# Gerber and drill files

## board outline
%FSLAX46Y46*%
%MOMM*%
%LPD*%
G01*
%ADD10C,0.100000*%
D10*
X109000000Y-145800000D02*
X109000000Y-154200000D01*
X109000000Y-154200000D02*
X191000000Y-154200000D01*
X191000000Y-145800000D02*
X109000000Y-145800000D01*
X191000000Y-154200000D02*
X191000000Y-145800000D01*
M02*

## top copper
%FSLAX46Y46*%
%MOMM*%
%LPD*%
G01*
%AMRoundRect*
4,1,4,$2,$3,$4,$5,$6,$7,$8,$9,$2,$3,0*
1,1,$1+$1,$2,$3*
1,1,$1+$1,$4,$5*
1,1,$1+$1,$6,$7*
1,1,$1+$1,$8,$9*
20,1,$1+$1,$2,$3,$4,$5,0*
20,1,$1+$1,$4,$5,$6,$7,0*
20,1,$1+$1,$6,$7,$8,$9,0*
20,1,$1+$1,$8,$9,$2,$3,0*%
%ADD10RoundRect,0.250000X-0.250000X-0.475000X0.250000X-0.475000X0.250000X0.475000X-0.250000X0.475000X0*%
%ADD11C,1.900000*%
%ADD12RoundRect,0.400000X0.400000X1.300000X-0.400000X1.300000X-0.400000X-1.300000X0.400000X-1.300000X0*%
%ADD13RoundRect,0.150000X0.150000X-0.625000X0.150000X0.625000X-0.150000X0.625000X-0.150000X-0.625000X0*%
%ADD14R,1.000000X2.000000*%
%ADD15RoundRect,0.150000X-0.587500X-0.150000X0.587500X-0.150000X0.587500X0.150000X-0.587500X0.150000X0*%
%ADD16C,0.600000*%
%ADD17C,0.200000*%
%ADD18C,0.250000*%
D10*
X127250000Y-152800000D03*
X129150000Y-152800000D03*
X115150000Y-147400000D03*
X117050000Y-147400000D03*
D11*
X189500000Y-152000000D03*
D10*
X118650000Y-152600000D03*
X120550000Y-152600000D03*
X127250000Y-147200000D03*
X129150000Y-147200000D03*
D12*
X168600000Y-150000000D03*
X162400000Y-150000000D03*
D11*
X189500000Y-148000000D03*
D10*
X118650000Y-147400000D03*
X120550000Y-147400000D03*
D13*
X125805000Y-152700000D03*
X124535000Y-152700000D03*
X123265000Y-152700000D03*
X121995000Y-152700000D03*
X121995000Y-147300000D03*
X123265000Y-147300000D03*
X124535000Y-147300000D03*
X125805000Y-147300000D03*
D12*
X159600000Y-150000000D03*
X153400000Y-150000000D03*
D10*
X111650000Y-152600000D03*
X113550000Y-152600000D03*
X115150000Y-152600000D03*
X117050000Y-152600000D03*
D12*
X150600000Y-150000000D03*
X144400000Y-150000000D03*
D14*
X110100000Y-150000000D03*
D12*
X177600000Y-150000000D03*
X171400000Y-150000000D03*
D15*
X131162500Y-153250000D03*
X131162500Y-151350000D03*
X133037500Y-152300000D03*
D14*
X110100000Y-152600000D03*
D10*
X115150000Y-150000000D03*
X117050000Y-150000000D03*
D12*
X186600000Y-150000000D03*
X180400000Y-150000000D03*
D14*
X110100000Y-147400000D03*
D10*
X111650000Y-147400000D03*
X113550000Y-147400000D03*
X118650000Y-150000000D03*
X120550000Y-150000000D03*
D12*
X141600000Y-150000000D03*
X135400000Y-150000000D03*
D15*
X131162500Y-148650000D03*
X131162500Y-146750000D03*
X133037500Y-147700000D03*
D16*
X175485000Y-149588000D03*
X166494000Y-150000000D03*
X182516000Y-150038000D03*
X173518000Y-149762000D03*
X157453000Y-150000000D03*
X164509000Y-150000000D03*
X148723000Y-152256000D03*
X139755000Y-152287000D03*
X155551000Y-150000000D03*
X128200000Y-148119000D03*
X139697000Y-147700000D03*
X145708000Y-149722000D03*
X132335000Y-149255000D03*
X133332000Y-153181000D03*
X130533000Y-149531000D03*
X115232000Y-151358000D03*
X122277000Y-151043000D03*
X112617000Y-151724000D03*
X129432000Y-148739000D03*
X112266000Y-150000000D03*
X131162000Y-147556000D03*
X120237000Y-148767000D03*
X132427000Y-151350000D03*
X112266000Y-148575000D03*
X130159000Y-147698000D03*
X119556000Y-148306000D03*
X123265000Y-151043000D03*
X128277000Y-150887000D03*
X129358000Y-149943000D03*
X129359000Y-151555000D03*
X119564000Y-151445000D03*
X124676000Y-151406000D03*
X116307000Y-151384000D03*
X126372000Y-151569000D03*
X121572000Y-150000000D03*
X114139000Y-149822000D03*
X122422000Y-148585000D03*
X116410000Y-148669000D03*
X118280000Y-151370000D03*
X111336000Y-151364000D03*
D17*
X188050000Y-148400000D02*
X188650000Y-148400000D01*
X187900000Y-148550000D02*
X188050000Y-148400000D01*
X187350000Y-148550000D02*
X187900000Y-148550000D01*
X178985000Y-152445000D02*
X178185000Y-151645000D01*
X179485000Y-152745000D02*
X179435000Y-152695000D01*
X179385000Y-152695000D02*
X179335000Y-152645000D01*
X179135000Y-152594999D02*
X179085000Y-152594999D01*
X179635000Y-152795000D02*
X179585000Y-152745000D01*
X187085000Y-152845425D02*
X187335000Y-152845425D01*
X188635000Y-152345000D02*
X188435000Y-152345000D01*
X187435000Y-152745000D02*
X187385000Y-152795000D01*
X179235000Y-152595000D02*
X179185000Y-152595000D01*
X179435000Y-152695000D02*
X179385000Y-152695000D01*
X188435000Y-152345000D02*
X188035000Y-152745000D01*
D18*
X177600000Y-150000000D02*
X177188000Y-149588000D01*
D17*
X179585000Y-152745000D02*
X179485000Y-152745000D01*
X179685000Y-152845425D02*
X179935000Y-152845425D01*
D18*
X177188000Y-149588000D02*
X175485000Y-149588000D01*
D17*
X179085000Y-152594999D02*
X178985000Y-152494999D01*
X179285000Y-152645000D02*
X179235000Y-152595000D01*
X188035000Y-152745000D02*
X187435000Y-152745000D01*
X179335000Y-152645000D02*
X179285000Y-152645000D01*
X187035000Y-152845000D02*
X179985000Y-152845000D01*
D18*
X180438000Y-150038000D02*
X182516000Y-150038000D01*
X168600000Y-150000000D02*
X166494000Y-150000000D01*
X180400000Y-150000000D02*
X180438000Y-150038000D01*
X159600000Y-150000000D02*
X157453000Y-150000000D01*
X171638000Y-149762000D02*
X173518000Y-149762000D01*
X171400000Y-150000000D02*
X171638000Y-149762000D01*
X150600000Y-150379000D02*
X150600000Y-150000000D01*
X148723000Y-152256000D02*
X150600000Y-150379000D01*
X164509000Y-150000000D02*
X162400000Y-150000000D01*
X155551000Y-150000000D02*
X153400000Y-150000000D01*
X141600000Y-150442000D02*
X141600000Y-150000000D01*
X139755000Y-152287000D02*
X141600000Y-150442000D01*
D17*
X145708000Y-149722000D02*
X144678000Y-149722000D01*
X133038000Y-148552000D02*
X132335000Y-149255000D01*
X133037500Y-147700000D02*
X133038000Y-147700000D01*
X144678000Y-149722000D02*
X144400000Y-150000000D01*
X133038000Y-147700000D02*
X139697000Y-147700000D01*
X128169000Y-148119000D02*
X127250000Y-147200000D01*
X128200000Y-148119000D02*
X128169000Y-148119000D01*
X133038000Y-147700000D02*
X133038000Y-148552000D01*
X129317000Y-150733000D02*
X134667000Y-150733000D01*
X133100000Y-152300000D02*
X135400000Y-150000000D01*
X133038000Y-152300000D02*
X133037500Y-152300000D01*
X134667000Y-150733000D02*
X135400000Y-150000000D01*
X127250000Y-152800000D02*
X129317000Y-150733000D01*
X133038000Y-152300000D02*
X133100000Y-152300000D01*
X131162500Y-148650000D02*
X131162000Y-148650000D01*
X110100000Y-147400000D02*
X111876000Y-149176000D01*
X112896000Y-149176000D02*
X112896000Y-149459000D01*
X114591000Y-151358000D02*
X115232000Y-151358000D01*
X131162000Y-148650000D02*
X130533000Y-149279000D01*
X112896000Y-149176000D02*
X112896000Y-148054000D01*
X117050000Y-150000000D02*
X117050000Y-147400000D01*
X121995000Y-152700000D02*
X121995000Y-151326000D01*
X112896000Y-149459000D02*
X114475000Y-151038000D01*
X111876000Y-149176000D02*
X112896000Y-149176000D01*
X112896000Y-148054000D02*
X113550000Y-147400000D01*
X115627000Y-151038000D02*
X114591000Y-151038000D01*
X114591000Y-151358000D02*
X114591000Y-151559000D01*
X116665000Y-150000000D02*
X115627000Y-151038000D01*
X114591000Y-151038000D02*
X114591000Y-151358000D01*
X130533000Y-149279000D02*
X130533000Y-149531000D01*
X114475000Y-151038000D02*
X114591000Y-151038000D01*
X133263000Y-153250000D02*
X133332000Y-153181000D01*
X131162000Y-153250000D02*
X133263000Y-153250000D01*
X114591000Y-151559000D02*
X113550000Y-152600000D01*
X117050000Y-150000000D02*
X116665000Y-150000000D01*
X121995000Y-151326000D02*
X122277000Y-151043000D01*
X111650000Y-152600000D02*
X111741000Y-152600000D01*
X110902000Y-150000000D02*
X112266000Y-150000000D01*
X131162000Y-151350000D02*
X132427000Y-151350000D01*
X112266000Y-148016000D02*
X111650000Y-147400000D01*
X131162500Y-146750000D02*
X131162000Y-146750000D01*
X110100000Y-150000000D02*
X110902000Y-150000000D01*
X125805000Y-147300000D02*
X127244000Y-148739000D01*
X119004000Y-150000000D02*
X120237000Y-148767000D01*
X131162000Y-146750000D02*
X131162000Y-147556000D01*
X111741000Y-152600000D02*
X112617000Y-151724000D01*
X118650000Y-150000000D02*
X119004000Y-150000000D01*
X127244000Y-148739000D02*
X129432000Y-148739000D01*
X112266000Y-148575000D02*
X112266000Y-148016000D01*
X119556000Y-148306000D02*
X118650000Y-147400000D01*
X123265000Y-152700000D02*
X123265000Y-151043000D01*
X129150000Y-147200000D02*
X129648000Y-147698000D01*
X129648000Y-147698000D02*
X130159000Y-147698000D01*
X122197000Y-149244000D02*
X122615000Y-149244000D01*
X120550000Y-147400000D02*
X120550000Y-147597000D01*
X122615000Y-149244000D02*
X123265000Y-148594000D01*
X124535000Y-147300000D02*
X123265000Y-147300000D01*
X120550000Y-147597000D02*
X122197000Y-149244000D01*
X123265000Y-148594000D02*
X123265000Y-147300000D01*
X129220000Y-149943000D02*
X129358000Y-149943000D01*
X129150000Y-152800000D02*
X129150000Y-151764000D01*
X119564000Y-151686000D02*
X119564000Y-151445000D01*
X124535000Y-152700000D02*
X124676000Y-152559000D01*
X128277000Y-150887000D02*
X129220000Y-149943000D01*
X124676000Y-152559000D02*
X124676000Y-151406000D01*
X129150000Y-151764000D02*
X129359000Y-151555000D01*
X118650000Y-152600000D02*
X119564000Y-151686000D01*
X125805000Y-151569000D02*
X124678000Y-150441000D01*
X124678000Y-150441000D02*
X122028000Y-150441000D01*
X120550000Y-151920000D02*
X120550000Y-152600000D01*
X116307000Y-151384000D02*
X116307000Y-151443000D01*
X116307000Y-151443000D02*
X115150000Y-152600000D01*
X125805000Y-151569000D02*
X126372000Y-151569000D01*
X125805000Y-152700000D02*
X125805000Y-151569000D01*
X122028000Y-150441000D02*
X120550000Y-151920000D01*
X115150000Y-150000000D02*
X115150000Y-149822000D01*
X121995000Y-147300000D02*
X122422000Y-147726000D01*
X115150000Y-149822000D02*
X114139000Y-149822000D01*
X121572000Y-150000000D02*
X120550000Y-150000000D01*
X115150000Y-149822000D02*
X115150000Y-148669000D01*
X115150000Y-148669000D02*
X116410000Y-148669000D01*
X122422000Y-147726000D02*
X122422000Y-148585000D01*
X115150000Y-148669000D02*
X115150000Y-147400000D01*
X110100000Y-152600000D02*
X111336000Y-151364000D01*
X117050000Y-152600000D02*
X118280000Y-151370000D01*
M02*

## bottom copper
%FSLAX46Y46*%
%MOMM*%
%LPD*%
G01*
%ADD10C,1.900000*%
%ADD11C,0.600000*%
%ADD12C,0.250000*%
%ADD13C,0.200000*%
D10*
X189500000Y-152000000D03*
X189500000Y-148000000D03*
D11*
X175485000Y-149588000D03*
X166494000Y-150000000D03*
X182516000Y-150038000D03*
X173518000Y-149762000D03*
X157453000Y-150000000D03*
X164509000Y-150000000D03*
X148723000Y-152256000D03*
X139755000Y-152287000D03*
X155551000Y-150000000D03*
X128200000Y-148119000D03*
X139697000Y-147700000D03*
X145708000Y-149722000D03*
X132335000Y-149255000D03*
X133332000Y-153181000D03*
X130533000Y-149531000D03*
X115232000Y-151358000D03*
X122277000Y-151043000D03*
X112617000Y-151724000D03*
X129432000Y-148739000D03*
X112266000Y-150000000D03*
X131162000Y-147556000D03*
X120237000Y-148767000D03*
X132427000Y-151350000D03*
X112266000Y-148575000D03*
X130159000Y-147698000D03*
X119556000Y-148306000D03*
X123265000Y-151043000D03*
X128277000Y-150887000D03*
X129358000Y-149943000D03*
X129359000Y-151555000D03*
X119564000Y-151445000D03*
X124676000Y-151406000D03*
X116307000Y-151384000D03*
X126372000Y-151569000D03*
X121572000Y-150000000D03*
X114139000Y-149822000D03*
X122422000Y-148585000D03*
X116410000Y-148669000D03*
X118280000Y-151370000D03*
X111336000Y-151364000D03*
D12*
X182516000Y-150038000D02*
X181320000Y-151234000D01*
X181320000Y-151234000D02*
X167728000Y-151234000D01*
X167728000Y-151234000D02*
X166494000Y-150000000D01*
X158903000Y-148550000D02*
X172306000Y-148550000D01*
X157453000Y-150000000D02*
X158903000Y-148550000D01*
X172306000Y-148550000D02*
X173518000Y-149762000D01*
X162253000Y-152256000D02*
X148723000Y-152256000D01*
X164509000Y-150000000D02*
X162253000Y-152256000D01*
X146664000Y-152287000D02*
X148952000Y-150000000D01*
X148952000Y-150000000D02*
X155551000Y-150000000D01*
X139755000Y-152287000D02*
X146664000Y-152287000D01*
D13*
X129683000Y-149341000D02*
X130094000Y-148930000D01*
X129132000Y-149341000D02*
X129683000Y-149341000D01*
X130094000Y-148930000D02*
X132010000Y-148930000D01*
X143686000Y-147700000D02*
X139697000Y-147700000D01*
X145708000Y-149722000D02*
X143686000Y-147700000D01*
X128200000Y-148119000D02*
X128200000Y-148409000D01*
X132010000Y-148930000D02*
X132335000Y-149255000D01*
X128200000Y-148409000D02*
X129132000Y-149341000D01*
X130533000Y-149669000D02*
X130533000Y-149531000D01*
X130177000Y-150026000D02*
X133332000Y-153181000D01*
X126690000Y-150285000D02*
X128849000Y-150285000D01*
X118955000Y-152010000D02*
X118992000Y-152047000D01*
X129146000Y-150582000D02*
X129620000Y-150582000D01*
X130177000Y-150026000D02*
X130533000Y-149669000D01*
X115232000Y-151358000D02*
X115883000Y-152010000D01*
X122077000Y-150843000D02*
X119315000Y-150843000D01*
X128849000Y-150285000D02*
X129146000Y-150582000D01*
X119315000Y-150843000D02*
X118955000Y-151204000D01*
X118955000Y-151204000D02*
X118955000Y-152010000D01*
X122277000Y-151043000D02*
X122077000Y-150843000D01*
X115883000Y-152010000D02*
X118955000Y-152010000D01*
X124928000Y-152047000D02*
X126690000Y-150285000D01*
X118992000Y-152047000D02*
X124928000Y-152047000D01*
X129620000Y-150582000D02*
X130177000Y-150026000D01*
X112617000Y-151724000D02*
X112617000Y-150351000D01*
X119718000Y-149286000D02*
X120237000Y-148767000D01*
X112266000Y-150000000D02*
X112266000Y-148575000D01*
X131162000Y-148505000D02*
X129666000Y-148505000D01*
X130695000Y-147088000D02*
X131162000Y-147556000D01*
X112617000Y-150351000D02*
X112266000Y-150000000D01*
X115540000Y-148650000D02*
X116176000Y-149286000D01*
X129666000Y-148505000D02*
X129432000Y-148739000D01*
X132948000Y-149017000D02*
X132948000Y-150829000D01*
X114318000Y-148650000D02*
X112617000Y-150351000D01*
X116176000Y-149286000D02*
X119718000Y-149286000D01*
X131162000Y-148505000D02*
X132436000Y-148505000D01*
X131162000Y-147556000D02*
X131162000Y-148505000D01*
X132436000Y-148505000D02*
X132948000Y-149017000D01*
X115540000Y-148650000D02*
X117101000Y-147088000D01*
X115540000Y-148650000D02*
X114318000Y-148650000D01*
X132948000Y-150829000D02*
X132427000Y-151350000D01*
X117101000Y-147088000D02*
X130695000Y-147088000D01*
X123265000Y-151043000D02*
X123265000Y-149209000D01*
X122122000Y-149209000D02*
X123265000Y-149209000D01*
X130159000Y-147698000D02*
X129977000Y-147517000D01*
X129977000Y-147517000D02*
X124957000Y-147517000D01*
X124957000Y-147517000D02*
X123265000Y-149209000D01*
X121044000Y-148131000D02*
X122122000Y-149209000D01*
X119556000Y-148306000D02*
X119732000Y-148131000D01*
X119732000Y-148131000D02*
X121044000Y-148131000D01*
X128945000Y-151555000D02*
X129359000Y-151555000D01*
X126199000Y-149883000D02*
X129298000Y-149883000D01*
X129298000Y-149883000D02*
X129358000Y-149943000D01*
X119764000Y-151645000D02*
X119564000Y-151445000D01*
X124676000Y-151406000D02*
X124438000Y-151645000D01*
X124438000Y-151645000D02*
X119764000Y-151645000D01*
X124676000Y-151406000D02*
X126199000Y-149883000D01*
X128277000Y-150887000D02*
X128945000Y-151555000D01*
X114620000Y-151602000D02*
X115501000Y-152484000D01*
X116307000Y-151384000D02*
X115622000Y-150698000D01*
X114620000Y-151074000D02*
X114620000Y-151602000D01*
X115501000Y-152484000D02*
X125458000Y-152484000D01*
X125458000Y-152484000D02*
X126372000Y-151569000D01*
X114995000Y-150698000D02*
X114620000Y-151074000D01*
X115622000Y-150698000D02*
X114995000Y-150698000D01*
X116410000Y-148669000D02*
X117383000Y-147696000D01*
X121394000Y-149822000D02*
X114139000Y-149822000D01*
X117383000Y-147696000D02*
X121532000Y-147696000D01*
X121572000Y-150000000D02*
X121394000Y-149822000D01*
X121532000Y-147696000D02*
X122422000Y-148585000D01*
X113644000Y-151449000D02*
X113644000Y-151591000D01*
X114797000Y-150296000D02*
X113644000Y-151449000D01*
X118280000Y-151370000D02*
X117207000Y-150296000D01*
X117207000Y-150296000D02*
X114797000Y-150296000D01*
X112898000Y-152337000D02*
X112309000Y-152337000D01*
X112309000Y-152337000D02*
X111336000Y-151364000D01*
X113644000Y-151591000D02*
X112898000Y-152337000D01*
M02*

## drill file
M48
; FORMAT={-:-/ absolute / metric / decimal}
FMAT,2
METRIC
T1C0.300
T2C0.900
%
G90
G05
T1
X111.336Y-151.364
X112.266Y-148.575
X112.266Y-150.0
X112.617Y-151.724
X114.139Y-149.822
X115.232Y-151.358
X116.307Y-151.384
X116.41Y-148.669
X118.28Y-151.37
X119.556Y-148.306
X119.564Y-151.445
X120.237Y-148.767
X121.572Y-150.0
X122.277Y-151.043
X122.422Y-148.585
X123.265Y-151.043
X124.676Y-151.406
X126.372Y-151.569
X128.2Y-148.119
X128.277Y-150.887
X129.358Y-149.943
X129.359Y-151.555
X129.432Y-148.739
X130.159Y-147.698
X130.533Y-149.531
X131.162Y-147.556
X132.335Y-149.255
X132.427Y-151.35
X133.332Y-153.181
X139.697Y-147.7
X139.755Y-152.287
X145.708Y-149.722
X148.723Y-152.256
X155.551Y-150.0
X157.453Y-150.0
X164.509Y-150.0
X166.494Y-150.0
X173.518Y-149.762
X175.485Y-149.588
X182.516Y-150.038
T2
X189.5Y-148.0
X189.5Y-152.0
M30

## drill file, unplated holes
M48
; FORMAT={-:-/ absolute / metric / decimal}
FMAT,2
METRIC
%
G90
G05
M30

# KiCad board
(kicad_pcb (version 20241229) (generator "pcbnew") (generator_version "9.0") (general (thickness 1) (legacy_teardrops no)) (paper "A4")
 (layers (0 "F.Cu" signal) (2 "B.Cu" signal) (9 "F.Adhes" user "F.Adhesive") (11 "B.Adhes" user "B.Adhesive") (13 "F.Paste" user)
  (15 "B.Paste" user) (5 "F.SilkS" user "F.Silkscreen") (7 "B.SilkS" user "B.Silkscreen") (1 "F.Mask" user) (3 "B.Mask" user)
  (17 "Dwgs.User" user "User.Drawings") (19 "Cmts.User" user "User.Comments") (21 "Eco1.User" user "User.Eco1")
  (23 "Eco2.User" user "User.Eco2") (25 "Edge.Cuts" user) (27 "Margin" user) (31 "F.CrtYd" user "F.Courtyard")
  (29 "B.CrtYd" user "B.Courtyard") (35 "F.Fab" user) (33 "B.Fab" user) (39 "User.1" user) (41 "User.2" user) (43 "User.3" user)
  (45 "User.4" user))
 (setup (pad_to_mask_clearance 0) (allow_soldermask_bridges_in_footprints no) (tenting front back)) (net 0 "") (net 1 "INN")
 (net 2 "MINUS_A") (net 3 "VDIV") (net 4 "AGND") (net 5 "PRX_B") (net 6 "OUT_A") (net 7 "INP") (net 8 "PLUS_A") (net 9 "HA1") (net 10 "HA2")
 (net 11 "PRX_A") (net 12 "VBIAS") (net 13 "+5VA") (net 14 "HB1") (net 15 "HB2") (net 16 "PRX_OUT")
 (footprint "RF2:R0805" (layer "F.Cu") (at 128.199999 152.8)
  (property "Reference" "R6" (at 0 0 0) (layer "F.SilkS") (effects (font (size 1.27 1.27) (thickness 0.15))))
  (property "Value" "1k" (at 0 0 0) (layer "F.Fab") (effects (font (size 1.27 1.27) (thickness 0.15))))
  (pad "1" smd roundrect (at -0.949999 0) (size 1 1.45) (layers "F.Cu" "F.Mask" "F.Paste") (roundrect_rratio 0.25) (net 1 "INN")
   (thermal_bridge_angle 45))
  (pad "2" smd roundrect (at 0.950001 0) (size 1 1.45) (layers "F.Cu" "F.Mask" "F.Paste") (roundrect_rratio 0.25) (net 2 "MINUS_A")
   (thermal_bridge_angle 45)))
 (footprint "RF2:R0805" (layer "F.Cu") (at 116.1 147.4)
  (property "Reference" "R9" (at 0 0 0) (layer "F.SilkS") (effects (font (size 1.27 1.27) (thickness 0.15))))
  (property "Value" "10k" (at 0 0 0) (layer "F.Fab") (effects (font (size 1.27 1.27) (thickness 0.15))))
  (pad "1" smd roundrect (at -0.95 0) (size 1 1.45) (layers "F.Cu" "F.Mask" "F.Paste") (roundrect_rratio 0.25) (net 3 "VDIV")
   (thermal_bridge_angle 45))
  (pad "2" smd roundrect (at 0.95 0) (size 1 1.45) (layers "F.Cu" "F.Mask" "F.Paste") (roundrect_rratio 0.25) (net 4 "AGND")
   (thermal_bridge_angle 45)))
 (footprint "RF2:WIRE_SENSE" (layer "F.Cu") (at 189.5 152)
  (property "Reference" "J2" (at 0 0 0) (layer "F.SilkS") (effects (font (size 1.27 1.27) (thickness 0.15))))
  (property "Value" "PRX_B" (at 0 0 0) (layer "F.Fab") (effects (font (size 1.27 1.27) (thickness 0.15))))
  (pad "1" thru_hole circle (at 0 0) (size 1.9 1.9) (drill 0.9) (layers "*.Cu" "*.Mask") (remove_unused_layers no) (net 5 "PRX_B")))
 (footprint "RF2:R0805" (layer "F.Cu") (at 119.6 152.6)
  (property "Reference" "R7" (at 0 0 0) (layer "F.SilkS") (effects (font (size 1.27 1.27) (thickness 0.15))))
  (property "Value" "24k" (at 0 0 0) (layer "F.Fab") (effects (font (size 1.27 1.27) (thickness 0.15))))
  (pad "1" smd roundrect (at -0.95 0) (size 1 1.45) (layers "F.Cu" "F.Mask" "F.Paste") (roundrect_rratio 0.25) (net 2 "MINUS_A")
   (thermal_bridge_angle 45))
  (pad "2" smd roundrect (at 0.95 0) (size 1 1.45) (layers "F.Cu" "F.Mask" "F.Paste") (roundrect_rratio 0.25) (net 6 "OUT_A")
   (thermal_bridge_angle 45)))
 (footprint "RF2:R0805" (layer "F.Cu") (at 128.199999 147.2)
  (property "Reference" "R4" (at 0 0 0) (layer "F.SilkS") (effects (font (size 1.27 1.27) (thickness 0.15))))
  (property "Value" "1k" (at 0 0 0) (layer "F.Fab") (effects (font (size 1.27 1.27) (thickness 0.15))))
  (pad "1" smd roundrect (at -0.949999 0) (size 1 1.45) (layers "F.Cu" "F.Mask" "F.Paste") (roundrect_rratio 0.25) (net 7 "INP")
   (thermal_bridge_angle 45))
  (pad "2" smd roundrect (at 0.950001 0) (size 1 1.45) (layers "F.Cu" "F.Mask" "F.Paste") (roundrect_rratio 0.25) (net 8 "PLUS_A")
   (thermal_bridge_angle 45)))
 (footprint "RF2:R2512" (layer "F.Cu") (at 165.5 150 180)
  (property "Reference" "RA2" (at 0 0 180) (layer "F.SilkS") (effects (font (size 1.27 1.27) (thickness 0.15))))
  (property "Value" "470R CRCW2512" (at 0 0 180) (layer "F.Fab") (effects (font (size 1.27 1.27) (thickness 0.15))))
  (pad "1" smd roundrect (at -3.1 0 180) (size 1.6 3.4) (layers "F.Cu" "F.Mask" "F.Paste") (roundrect_rratio 0.25) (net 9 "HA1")
   (thermal_bridge_angle 45))
  (pad "2" smd roundrect (at 3.1 0 180) (size 1.6 3.4) (layers "F.Cu" "F.Mask" "F.Paste") (roundrect_rratio 0.25) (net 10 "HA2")
   (thermal_bridge_angle 45)))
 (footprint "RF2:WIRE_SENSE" (layer "F.Cu") (at 189.5 148)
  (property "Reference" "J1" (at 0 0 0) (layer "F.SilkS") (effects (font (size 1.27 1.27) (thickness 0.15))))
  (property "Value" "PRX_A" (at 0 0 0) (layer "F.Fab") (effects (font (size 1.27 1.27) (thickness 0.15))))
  (pad "1" thru_hole circle (at 0 0) (size 1.9 1.9) (drill 0.9) (layers "*.Cu" "*.Mask") (remove_unused_layers no) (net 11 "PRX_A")))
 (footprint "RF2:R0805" (layer "F.Cu") (at 119.6 147.4)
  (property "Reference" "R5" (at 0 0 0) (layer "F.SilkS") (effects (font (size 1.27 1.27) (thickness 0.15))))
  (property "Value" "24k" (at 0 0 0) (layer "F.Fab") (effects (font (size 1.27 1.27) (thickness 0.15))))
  (pad "1" smd roundrect (at -0.95 0) (size 1 1.45) (layers "F.Cu" "F.Mask" "F.Paste") (roundrect_rratio 0.25) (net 8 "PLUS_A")
   (thermal_bridge_angle 45))
  (pad "2" smd roundrect (at 0.95 0) (size 1 1.45) (layers "F.Cu" "F.Mask" "F.Paste") (roundrect_rratio 0.25) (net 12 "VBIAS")
   (thermal_bridge_angle 45)))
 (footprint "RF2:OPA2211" (layer "F.Cu") (at 123.9 150 90)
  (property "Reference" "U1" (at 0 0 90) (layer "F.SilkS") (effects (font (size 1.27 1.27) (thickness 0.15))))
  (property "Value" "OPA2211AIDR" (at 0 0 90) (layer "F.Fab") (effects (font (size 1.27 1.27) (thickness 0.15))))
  (pad "1" smd roundrect (at -2.7 1.905 90) (size 1.55 0.6) (layers "F.Cu" "F.Mask" "F.Paste") (roundrect_rratio 0.25) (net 6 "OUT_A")
   (thermal_bridge_angle 45))
  (pad "2" smd roundrect (at -2.7 0.635 90) (size 1.55 0.6) (layers "F.Cu" "F.Mask" "F.Paste") (roundrect_rratio 0.25) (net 2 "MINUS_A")
   (thermal_bridge_angle 45))
  (pad "3" smd roundrect (at -2.7 -0.635 90) (size 1.55 0.6) (layers "F.Cu" "F.Mask" "F.Paste") (roundrect_rratio 0.25) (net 8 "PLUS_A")
   (thermal_bridge_angle 45))
  (pad "4" smd roundrect (at -2.7 -1.905 90) (size 1.55 0.6) (layers "F.Cu" "F.Mask" "F.Paste") (roundrect_rratio 0.25) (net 4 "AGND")
   (thermal_bridge_angle 45))
  (pad "5" smd roundrect (at 2.7 -1.905 90) (size 1.55 0.6) (layers "F.Cu" "F.Mask" "F.Paste") (roundrect_rratio 0.25) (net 3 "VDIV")
   (thermal_bridge_angle 45))
  (pad "6" smd roundrect (at 2.7 -0.635 90) (size 1.55 0.6) (layers "F.Cu" "F.Mask" "F.Paste") (roundrect_rratio 0.25) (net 12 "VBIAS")
   (thermal_bridge_angle 45))
  (pad "7" smd roundrect (at 2.7 0.635 90) (size 1.55 0.6) (layers "F.Cu" "F.Mask" "F.Paste") (roundrect_rratio 0.25) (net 12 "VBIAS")
   (thermal_bridge_angle 45))
  (pad "8" smd roundrect (at 2.7 1.905 90) (size 1.55 0.6) (layers "F.Cu" "F.Mask" "F.Paste") (roundrect_rratio 0.25) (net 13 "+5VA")
   (thermal_bridge_angle 45)))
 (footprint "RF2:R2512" (layer "F.Cu") (at 156.5 150 180)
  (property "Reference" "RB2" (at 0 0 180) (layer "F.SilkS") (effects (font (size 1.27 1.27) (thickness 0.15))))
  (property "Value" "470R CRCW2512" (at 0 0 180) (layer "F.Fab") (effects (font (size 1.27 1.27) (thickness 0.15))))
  (pad "1" smd roundrect (at -3.1 0 180) (size 1.6 3.4) (layers "F.Cu" "F.Mask" "F.Paste") (roundrect_rratio 0.25) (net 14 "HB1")
   (thermal_bridge_angle 45))
  (pad "2" smd roundrect (at 3.1 0 180) (size 1.6 3.4) (layers "F.Cu" "F.Mask" "F.Paste") (roundrect_rratio 0.25) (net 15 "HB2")
   (thermal_bridge_angle 45)))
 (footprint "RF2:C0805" (layer "F.Cu") (at 112.6 152.6)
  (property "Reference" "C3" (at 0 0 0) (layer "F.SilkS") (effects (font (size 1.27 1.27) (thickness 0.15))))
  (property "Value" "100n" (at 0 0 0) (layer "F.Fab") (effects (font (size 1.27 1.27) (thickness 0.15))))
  (pad "1" smd roundrect (at -0.95 0) (size 1 1.45) (layers "F.Cu" "F.Mask" "F.Paste") (roundrect_rratio 0.25) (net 13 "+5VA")
   (thermal_bridge_angle 45))
  (pad "2" smd roundrect (at 0.95 0) (size 1 1.45) (layers "F.Cu" "F.Mask" "F.Paste") (roundrect_rratio 0.25) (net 4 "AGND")
   (thermal_bridge_angle 45)))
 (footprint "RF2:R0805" (layer "F.Cu") (at 116.1 152.6)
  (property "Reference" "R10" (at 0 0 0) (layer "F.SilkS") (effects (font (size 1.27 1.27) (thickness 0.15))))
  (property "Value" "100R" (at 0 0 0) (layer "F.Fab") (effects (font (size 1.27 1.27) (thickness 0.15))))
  (pad "1" smd roundrect (at -0.95 0) (size 1 1.45) (layers "F.Cu" "F.Mask" "F.Paste") (roundrect_rratio 0.25) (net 6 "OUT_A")
   (thermal_bridge_angle 45))
  (pad "2" smd roundrect (at 0.95 0) (size 1 1.45) (layers "F.Cu" "F.Mask" "F.Paste") (roundrect_rratio 0.25) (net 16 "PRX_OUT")
   (thermal_bridge_angle 45)))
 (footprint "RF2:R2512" (layer "F.Cu") (at 147.5 150 180)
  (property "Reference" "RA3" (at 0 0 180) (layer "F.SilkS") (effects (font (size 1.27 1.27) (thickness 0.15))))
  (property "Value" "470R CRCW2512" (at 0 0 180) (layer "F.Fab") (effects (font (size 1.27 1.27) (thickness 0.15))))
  (pad "1" smd roundrect (at -3.1 0 180) (size 1.6 3.4) (layers "F.Cu" "F.Mask" "F.Paste") (roundrect_rratio 0.25) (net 10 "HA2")
   (thermal_bridge_angle 45))
  (pad "2" smd roundrect (at 3.1 0 180) (size 1.6 3.4) (layers "F.Cu" "F.Mask" "F.Paste") (roundrect_rratio 0.25) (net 7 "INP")
   (thermal_bridge_angle 45)))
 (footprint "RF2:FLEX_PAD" (layer "F.Cu") (at 110.1 150)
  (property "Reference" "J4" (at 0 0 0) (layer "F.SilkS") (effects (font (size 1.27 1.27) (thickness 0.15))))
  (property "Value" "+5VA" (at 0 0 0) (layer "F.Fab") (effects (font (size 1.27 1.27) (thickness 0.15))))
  (pad "1" smd rect (at 0 0) (size 1 2) (layers "F.Cu" "F.Mask" "F.Paste") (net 13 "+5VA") (thermal_bridge_angle 45)))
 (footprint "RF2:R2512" (layer "F.Cu") (at 174.5 150 180)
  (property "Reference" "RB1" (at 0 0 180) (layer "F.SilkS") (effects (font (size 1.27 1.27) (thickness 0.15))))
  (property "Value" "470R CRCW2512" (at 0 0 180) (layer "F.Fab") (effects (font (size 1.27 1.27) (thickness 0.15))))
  (pad "1" smd roundrect (at -3.1 0 180) (size 1.6 3.4) (layers "F.Cu" "F.Mask" "F.Paste") (roundrect_rratio 0.25) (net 5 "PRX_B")
   (thermal_bridge_angle 45))
  (pad "2" smd roundrect (at 3.1 0 180) (size 1.6 3.4) (layers "F.Cu" "F.Mask" "F.Paste") (roundrect_rratio 0.25) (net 14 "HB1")
   (thermal_bridge_angle 45)))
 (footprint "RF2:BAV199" (layer "F.Cu") (at 132.1 152.3)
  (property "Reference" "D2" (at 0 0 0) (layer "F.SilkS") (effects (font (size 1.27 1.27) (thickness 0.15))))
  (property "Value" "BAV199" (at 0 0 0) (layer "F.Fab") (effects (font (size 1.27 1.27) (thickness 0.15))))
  (pad "1" smd roundrect (at -0.9375 0.95) (size 1.475 0.6) (layers "F.Cu" "F.Mask" "F.Paste") (roundrect_rratio 0.25) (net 4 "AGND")
   (thermal_bridge_angle 45))
  (pad "2" smd roundrect (at -0.9375 -0.95) (size 1.475 0.6) (layers "F.Cu" "F.Mask" "F.Paste") (roundrect_rratio 0.25) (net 13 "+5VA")
   (thermal_bridge_angle 45))
  (pad "3" smd roundrect (at 0.9375 0) (size 1.475 0.6) (layers "F.Cu" "F.Mask" "F.Paste") (roundrect_rratio 0.25) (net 1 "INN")
   (thermal_bridge_angle 45)))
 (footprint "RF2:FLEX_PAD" (layer "F.Cu") (at 110.1 152.6)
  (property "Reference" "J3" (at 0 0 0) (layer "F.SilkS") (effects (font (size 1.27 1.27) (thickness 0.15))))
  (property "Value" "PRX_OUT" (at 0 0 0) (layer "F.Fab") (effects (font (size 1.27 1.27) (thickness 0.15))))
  (pad "1" smd rect (at 0 0) (size 1 2) (layers "F.Cu" "F.Mask" "F.Paste") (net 16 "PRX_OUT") (thermal_bridge_angle 45)))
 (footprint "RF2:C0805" (layer "F.Cu") (at 116.1 150)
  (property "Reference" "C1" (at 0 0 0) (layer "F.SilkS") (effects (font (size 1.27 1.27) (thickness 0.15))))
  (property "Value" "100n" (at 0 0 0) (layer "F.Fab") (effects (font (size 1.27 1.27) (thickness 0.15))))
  (pad "1" smd roundrect (at -0.95 0) (size 1 1.45) (layers "F.Cu" "F.Mask" "F.Paste") (roundrect_rratio 0.25) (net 3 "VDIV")
   (thermal_bridge_angle 45))
  (pad "2" smd roundrect (at 0.95 0) (size 1 1.45) (layers "F.Cu" "F.Mask" "F.Paste") (roundrect_rratio 0.25) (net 4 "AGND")
   (thermal_bridge_angle 45)))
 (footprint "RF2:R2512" (layer "F.Cu") (at 183.5 150 180)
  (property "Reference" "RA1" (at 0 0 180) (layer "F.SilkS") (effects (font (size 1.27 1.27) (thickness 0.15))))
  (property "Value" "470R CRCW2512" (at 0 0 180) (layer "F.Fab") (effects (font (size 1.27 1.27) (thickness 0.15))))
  (pad "1" smd roundrect (at -3.1 0 180) (size 1.6 3.4) (layers "F.Cu" "F.Mask" "F.Paste") (roundrect_rratio 0.25) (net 11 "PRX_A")
   (thermal_bridge_angle 45))
  (pad "2" smd roundrect (at 3.1 0 180) (size 1.6 3.4) (layers "F.Cu" "F.Mask" "F.Paste") (roundrect_rratio 0.25) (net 9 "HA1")
   (thermal_bridge_angle 45)))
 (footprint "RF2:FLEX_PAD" (layer "F.Cu") (at 110.1 147.4)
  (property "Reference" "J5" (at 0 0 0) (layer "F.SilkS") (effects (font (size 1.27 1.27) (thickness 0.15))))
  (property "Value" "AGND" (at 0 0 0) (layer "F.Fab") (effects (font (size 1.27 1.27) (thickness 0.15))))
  (pad "1" smd rect (at 0 0) (size 1 2) (layers "F.Cu" "F.Mask" "F.Paste") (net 4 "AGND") (thermal_bridge_angle 45)))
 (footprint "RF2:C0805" (layer "F.Cu") (at 112.6 147.4)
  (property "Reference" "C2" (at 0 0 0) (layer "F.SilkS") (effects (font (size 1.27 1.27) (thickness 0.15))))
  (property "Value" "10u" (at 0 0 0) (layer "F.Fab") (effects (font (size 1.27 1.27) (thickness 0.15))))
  (pad "1" smd roundrect (at -0.95 0) (size 1 1.45) (layers "F.Cu" "F.Mask" "F.Paste") (roundrect_rratio 0.25) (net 13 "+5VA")
   (thermal_bridge_angle 45))
  (pad "2" smd roundrect (at 0.95 0) (size 1 1.45) (layers "F.Cu" "F.Mask" "F.Paste") (roundrect_rratio 0.25) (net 4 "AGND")
   (thermal_bridge_angle 45)))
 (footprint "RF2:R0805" (layer "F.Cu") (at 119.6 150)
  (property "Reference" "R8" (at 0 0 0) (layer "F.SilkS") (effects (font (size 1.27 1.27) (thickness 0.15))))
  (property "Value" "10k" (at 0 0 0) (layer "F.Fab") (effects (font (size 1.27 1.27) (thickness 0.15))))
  (pad "1" smd roundrect (at -0.95 0) (size 1 1.45) (layers "F.Cu" "F.Mask" "F.Paste") (roundrect_rratio 0.25) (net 13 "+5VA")
   (thermal_bridge_angle 45))
  (pad "2" smd roundrect (at 0.95 0) (size 1 1.45) (layers "F.Cu" "F.Mask" "F.Paste") (roundrect_rratio 0.25) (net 3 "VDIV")
   (thermal_bridge_angle 45)))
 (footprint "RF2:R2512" (layer "F.Cu") (at 138.5 150 180)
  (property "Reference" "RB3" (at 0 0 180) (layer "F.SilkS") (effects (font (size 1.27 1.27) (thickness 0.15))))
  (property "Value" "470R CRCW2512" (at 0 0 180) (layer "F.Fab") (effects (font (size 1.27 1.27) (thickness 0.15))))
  (pad "1" smd roundrect (at -3.1 0 180) (size 1.6 3.4) (layers "F.Cu" "F.Mask" "F.Paste") (roundrect_rratio 0.25) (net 15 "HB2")
   (thermal_bridge_angle 45))
  (pad "2" smd roundrect (at 3.1 0 180) (size 1.6 3.4) (layers "F.Cu" "F.Mask" "F.Paste") (roundrect_rratio 0.25) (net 1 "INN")
   (thermal_bridge_angle 45)))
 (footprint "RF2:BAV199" (layer "F.Cu") (at 132.1 147.7)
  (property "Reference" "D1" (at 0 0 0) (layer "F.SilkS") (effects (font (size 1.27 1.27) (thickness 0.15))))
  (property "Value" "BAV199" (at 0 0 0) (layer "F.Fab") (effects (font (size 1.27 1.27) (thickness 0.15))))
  (pad "1" smd roundrect (at -0.9375 0.95) (size 1.475 0.6) (layers "F.Cu" "F.Mask" "F.Paste") (roundrect_rratio 0.25) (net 4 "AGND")
   (thermal_bridge_angle 45))
  (pad "2" smd roundrect (at -0.9375 -0.95) (size 1.475 0.6) (layers "F.Cu" "F.Mask" "F.Paste") (roundrect_rratio 0.25) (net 13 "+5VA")
   (thermal_bridge_angle 45))
  (pad "3" smd roundrect (at 0.9375 0) (size 1.475 0.6) (layers "F.Cu" "F.Mask" "F.Paste") (roundrect_rratio 0.25) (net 7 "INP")
   (thermal_bridge_angle 45)))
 (gr_line (start 109 145.8) (end 109 154.2) (stroke (width 0.1) (type default)) (layer "Edge.Cuts"))
 (gr_line (start 109 154.2) (end 191 154.2) (stroke (width 0.1) (type default)) (layer "Edge.Cuts"))
 (gr_line (start 191 145.8) (end 109 145.8) (stroke (width 0.1) (type default)) (layer "Edge.Cuts"))
 (gr_line (start 191 154.2) (end 191 145.8) (stroke (width 0.1) (type default)) (layer "Edge.Cuts"))
 (segment (start 188.05 148.4) (end 188.65 148.4) (width 0.2) (layer "F.Cu") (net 11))
 (segment (start 187.9 148.55) (end 188.05 148.4) (width 0.2) (layer "F.Cu") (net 11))
 (segment (start 187.35 148.55) (end 187.9 148.55) (width 0.2) (layer "F.Cu") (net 11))
 (segment (start 178.985 152.445) (end 178.185 151.645) (width 0.2) (layer "F.Cu") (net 5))
 (segment (start 179.485 152.745) (end 179.435 152.695) (width 0.2) (layer "F.Cu") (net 5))
 (segment (start 179.385 152.695) (end 179.335 152.645) (width 0.2) (layer "F.Cu") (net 5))
 (segment (start 179.135 152.594999) (end 179.085 152.594999) (width 0.2) (layer "F.Cu") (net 5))
 (segment (start 179.635 152.795) (end 179.585 152.745) (width 0.2) (layer "F.Cu") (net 5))
 (segment (start 187.085 152.845425) (end 187.335 152.845425) (width 0.2) (layer "F.Cu") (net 5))
 (segment (start 188.635 152.345) (end 188.435 152.345) (width 0.2) (layer "F.Cu") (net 5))
 (segment (start 187.435 152.745) (end 187.385 152.795) (width 0.2) (layer "F.Cu") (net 5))
 (segment (start 179.235 152.595) (end 179.185 152.595) (width 0.2) (layer "F.Cu") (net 5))
 (segment (start 179.435 152.695) (end 179.385 152.695) (width 0.2) (layer "F.Cu") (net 5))
 (segment (start 188.435 152.345) (end 188.035 152.745) (width 0.2) (layer "F.Cu") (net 5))
 (segment (start 177.6 150) (end 177.188 149.588) (width 0.25) (layer "F.Cu") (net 5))
 (segment (start 179.585 152.745) (end 179.485 152.745) (width 0.2) (layer "F.Cu") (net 5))
 (segment (start 179.685 152.845425) (end 179.935 152.845425) (width 0.2) (layer "F.Cu") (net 5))
 (segment (start 177.188 149.588) (end 175.485 149.588) (width 0.25) (layer "F.Cu") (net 5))
 (segment (start 179.085 152.594999) (end 178.985 152.494999) (width 0.2) (layer "F.Cu") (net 5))
 (segment (start 179.285 152.645) (end 179.235 152.595) (width 0.2) (layer "F.Cu") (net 5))
 (segment (start 188.035 152.745) (end 187.435 152.745) (width 0.2) (layer "F.Cu") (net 5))
 (segment (start 179.335 152.645) (end 179.285 152.645) (width 0.2) (layer "F.Cu") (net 5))
 (segment (start 187.035 152.845) (end 179.985 152.845) (width 0.2) (layer "F.Cu") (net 5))
 (via (at 175.485 149.588) (size 0.6) (drill 0.3) (layers "F.Cu" "B.Cu") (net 5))
 (segment (start 180.438 150.038) (end 182.516 150.038) (width 0.25) (layer "F.Cu") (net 9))
 (segment (start 168.6 150) (end 166.494 150) (width 0.25) (layer "F.Cu") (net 9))
 (segment (start 180.4 150) (end 180.438 150.038) (width 0.25) (layer "F.Cu") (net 9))
 (via (at 166.494 150) (size 0.6) (drill 0.3) (layers "F.Cu" "B.Cu") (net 9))
 (via (at 182.516 150.038) (size 0.6) (drill 0.3) (layers "F.Cu" "B.Cu") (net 9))
 (segment (start 182.516 150.038) (end 181.32 151.234) (width 0.25) (layer "B.Cu") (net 9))
 (segment (start 181.32 151.234) (end 167.728 151.234) (width 0.25) (layer "B.Cu") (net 9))
 (segment (start 167.728 151.234) (end 166.494 150) (width 0.25) (layer "B.Cu") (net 9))
 (segment (start 159.6 150) (end 157.453 150) (width 0.25) (layer "F.Cu") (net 14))
 (segment (start 171.638 149.762) (end 173.518 149.762) (width 0.25) (layer "F.Cu") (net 14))
 (segment (start 171.4 150) (end 171.638 149.762) (width 0.25) (layer "F.Cu") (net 14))
 (via (at 173.518 149.762) (size 0.6) (drill 0.3) (layers "F.Cu" "B.Cu") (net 14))
 (via (at 157.453 150) (size 0.6) (drill 0.3) (layers "F.Cu" "B.Cu") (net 14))
 (segment (start 158.903 148.55) (end 172.306 148.55) (width 0.25) (layer "B.Cu") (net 14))
 (segment (start 157.453 150) (end 158.903 148.55) (width 0.25) (layer "B.Cu") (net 14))
 (segment (start 172.306 148.55) (end 173.518 149.762) (width 0.25) (layer "B.Cu") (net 14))
 (segment (start 150.6 150.379) (end 150.6 150) (width 0.25) (layer "F.Cu") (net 10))
 (segment (start 148.723 152.256) (end 150.6 150.379) (width 0.25) (layer "F.Cu") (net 10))
 (segment (start 164.509 150) (end 162.4 150) (width 0.25) (layer "F.Cu") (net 10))
 (via (at 164.509 150) (size 0.6) (drill 0.3) (layers "F.Cu" "B.Cu") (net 10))
 (via (at 148.723 152.256) (size 0.6) (drill 0.3) (layers "F.Cu" "B.Cu") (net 10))
 (segment (start 162.253 152.256) (end 148.723 152.256) (width 0.25) (layer "B.Cu") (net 10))
 (segment (start 164.509 150) (end 162.253 152.256) (width 0.25) (layer "B.Cu") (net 10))
 (segment (start 155.551 150) (end 153.4 150) (width 0.25) (layer "F.Cu") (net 15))
 (segment (start 141.6 150.442) (end 141.6 150) (width 0.25) (layer "F.Cu") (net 15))
 (segment (start 139.755 152.287) (end 141.6 150.442) (width 0.25) (layer "F.Cu") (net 15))
 (via (at 139.755 152.287) (size 0.6) (drill 0.3) (layers "F.Cu" "B.Cu") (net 15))
 (via (at 155.551 150) (size 0.6) (drill 0.3) (layers "F.Cu" "B.Cu") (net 15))
 (segment (start 146.664 152.287) (end 148.952 150) (width 0.25) (layer "B.Cu") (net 15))
 (segment (start 148.952 150) (end 155.551 150) (width 0.25) (layer "B.Cu") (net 15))
 (segment (start 139.755 152.287) (end 146.664 152.287) (width 0.25) (layer "B.Cu") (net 15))
 (segment (start 145.708 149.722) (end 144.678 149.722) (width 0.2) (layer "F.Cu") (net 7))
 (segment (start 133.038 148.552) (end 132.335 149.255) (width 0.2) (layer "F.Cu") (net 7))
 (segment (start 133.0375 147.7) (end 133.038 147.7) (width 0.2) (layer "F.Cu") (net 7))
 (segment (start 144.678 149.722) (end 144.4 150) (width 0.2) (layer "F.Cu") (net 7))
 (segment (start 133.038 147.7) (end 139.697 147.7) (width 0.2) (layer "F.Cu") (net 7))
 (segment (start 128.169 148.119) (end 127.25 147.2) (width 0.2) (layer "F.Cu") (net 7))
 (segment (start 128.2 148.119) (end 128.169 148.119) (width 0.2) (layer "F.Cu") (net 7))
 (segment (start 133.038 147.7) (end 133.038 148.552) (width 0.2) (layer "F.Cu") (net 7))
 (via (at 128.2 148.119) (size 0.6) (drill 0.3) (layers "F.Cu" "B.Cu") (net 7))
 (via (at 139.697 147.7) (size 0.6) (drill 0.3) (layers "F.Cu" "B.Cu") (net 7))
 (via (at 145.708 149.722) (size 0.6) (drill 0.3) (layers "F.Cu" "B.Cu") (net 7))
 (via (at 132.335 149.255) (size 0.6) (drill 0.3) (layers "F.Cu" "B.Cu") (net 7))
 (segment (start 129.683 149.341) (end 130.094 148.93) (width 0.2) (layer "B.Cu") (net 7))
 (segment (start 129.132 149.341) (end 129.683 149.341) (width 0.2) (layer "B.Cu") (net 7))
 (segment (start 130.094 148.93) (end 132.01 148.93) (width 0.2) (layer "B.Cu") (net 7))
 (segment (start 143.686 147.7) (end 139.697 147.7) (width 0.2) (layer "B.Cu") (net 7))
 (segment (start 145.708 149.722) (end 143.686 147.7) (width 0.2) (layer "B.Cu") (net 7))
 (segment (start 128.2 148.119) (end 128.2 148.409) (width 0.2) (layer "B.Cu") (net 7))
 (segment (start 132.01 148.93) (end 132.335 149.255) (width 0.2) (layer "B.Cu") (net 7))
 (segment (start 128.2 148.409) (end 129.132 149.341) (width 0.2) (layer "B.Cu") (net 7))
 (segment (start 129.317 150.733) (end 134.667 150.733) (width 0.2) (layer "F.Cu") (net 1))
 (segment (start 133.1 152.3) (end 135.4 150) (width 0.2) (layer "F.Cu") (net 1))
 (segment (start 133.038 152.3) (end 133.0375 152.3) (width 0.2) (layer "F.Cu") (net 1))
 (segment (start 134.667 150.733) (end 135.4 150) (width 0.2) (layer "F.Cu") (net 1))
 (segment (start 127.25 152.8) (end 129.317 150.733) (width 0.2) (layer "F.Cu") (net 1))
 (segment (start 133.038 152.3) (end 133.1 152.3) (width 0.2) (layer "F.Cu") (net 1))
 (segment (start 131.1625 148.65) (end 131.162 148.65) (width 0.2) (layer "F.Cu") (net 4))
 (segment (start 110.1 147.4) (end 111.876 149.176) (width 0.2) (layer "F.Cu") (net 4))
 (segment (start 112.896 149.176) (end 112.896 149.459) (width 0.2) (layer "F.Cu") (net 4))
 (segment (start 114.591 151.358) (end 115.232 151.358) (width 0.2) (layer "F.Cu") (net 4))
 (segment (start 131.162 148.65) (end 130.533 149.279) (width 0.2) (layer "F.Cu") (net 4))
 (segment (start 112.896 149.176) (end 112.896 148.054) (width 0.2) (layer "F.Cu") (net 4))
 (segment (start 117.05 150) (end 117.05 147.4) (width 0.2) (layer "F.Cu") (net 4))
 (segment (start 121.995 152.7) (end 121.995 151.326) (width 0.2) (layer "F.Cu") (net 4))
 (segment (start 112.896 149.459) (end 114.475 151.038) (width 0.2) (layer "F.Cu") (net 4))
 (segment (start 111.876 149.176) (end 112.896 149.176) (width 0.2) (layer "F.Cu") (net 4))
 (segment (start 112.896 148.054) (end 113.55 147.4) (width 0.2) (layer "F.Cu") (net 4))
 (segment (start 115.627 151.038) (end 114.591 151.038) (width 0.2) (layer "F.Cu") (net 4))
 (segment (start 114.591 151.358) (end 114.591 151.559) (width 0.2) (layer "F.Cu") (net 4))
 (segment (start 116.665 150) (end 115.627 151.038) (width 0.2) (layer "F.Cu") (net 4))
 (segment (start 114.591 151.038) (end 114.591 151.358) (width 0.2) (layer "F.Cu") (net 4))
 (segment (start 130.533 149.279) (end 130.533 149.531) (width 0.2) (layer "F.Cu") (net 4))
 (segment (start 114.475 151.038) (end 114.591 151.038) (width 0.2) (layer "F.Cu") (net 4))
 (segment (start 133.263 153.25) (end 133.332 153.181) (width 0.2) (layer "F.Cu") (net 4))
 (segment (start 131.162 153.25) (end 133.263 153.25) (width 0.2) (layer "F.Cu") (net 4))
 (segment (start 114.591 151.559) (end 113.55 152.6) (width 0.2) (layer "F.Cu") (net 4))
 (segment (start 117.05 150) (end 116.665 150) (width 0.2) (layer "F.Cu") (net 4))
 (segment (start 121.995 151.326) (end 122.277 151.043) (width 0.2) (layer "F.Cu") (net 4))
 (via (at 133.332 153.181) (size 0.6) (drill 0.3) (layers "F.Cu" "B.Cu") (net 4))
 (via (at 130.533 149.531) (size 0.6) (drill 0.3) (layers "F.Cu" "B.Cu") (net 4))
 (via (at 115.232 151.358) (size 0.6) (drill 0.3) (layers "F.Cu" "B.Cu") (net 4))
 (via (at 122.277 151.043) (size 0.6) (drill 0.3) (layers "F.Cu" "B.Cu") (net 4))
 (segment (start 130.533 149.669) (end 130.533 149.531) (width 0.2) (layer "B.Cu") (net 4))
 (segment (start 130.177 150.026) (end 133.332 153.181) (width 0.2) (layer "B.Cu") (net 4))
 (segment (start 126.69 150.285) (end 128.849 150.285) (width 0.2) (layer "B.Cu") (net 4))
 (segment (start 118.955 152.01) (end 118.992 152.047) (width 0.2) (layer "B.Cu") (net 4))
 (segment (start 129.146 150.582) (end 129.62 150.582) (width 0.2) (layer "B.Cu") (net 4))
 (segment (start 130.177 150.026) (end 130.533 149.669) (width 0.2) (layer "B.Cu") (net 4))
 (segment (start 115.232 151.358) (end 115.883 152.01) (width 0.2) (layer "B.Cu") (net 4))
 (segment (start 122.077 150.843) (end 119.315 150.843) (width 0.2) (layer "B.Cu") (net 4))
 (segment (start 128.849 150.285) (end 129.146 150.582) (width 0.2) (layer "B.Cu") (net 4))
 (segment (start 119.315 150.843) (end 118.955 151.204) (width 0.2) (layer "B.Cu") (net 4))
 (segment (start 118.955 151.204) (end 118.955 152.01) (width 0.2) (layer "B.Cu") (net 4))
 (segment (start 122.277 151.043) (end 122.077 150.843) (width 0.2) (layer "B.Cu") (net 4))
 (segment (start 115.883 152.01) (end 118.955 152.01) (width 0.2) (layer "B.Cu") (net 4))
 (segment (start 124.928 152.047) (end 126.69 150.285) (width 0.2) (layer "B.Cu") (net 4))
 (segment (start 118.992 152.047) (end 124.928 152.047) (width 0.2) (layer "B.Cu") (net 4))
 (segment (start 129.62 150.582) (end 130.177 150.026) (width 0.2) (layer "B.Cu") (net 4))
 (segment (start 111.65 152.6) (end 111.741 152.6) (width 0.2) (layer "F.Cu") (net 13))
 (segment (start 110.902 150) (end 112.266 150) (width 0.2) (layer "F.Cu") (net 13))
 (segment (start 131.162 151.35) (end 132.427 151.35) (width 0.2) (layer "F.Cu") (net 13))
 (segment (start 112.266 148.016) (end 111.65 147.4) (width 0.2) (layer "F.Cu") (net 13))
 (segment (start 131.1625 146.75) (end 131.162 146.75) (width 0.2) (layer "F.Cu") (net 13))
 (segment (start 110.1 150) (end 110.902 150) (width 0.2) (layer "F.Cu") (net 13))
 (segment (start 125.805 147.3) (end 127.244 148.739) (width 0.2) (layer "F.Cu") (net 13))
 (segment (start 119.004 150) (end 120.237 148.767) (width 0.2) (layer "F.Cu") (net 13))
 (segment (start 131.162 146.75) (end 131.162 147.556) (width 0.2) (layer "F.Cu") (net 13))
 (segment (start 111.741 152.6) (end 112.617 151.724) (width 0.2) (layer "F.Cu") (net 13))
 (segment (start 118.65 150) (end 119.004 150) (width 0.2) (layer "F.Cu") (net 13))
 (segment (start 127.244 148.739) (end 129.432 148.739) (width 0.2) (layer "F.Cu") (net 13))
 (segment (start 112.266 148.575) (end 112.266 148.016) (width 0.2) (layer "F.Cu") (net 13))
 (via (at 112.617 151.724) (size 0.6) (drill 0.3) (layers "F.Cu" "B.Cu") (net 13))
 (via (at 129.432 148.739) (size 0.6) (drill 0.3) (layers "F.Cu" "B.Cu") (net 13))
 (via (at 112.266 150) (size 0.6) (drill 0.3) (layers "F.Cu" "B.Cu") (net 13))
 (via (at 131.162 147.556) (size 0.6) (drill 0.3) (layers "F.Cu" "B.Cu") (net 13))
 (via (at 120.237 148.767) (size 0.6) (drill 0.3) (layers "F.Cu" "B.Cu") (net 13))
 (via (at 132.427 151.35) (size 0.6) (drill 0.3) (layers "F.Cu" "B.Cu") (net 13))
 (via (at 112.266 148.575) (size 0.6) (drill 0.3) (layers "F.Cu" "B.Cu") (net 13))
 (segment (start 112.617 151.724) (end 112.617 150.351) (width 0.2) (layer "B.Cu") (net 13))
 (segment (start 119.718 149.286) (end 120.237 148.767) (width 0.2) (layer "B.Cu") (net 13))
 (segment (start 112.266 150) (end 112.266 148.575) (width 0.2) (layer "B.Cu") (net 13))
 (segment (start 131.162 148.505) (end 129.666 148.505) (width 0.2) (layer "B.Cu") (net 13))
 (segment (start 130.695 147.088) (end 131.162 147.556) (width 0.2) (layer "B.Cu") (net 13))
 (segment (start 112.617 150.351) (end 112.266 150) (width 0.2) (layer "B.Cu") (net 13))
 (segment (start 115.54 148.65) (end 116.176 149.286) (width 0.2) (layer "B.Cu") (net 13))
 (segment (start 129.666 148.505) (end 129.432 148.739) (width 0.2) (layer "B.Cu") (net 13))
 (segment (start 132.948 149.017) (end 132.948 150.829) (width 0.2) (layer "B.Cu") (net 13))
 (segment (start 114.318 148.65) (end 112.617 150.351) (width 0.2) (layer "B.Cu") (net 13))
 (segment (start 116.176 149.286) (end 119.718 149.286) (width 0.2) (layer "B.Cu") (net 13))
 (segment (start 131.162 148.505) (end 132.436 148.505) (width 0.2) (layer "B.Cu") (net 13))
 (segment (start 131.162 147.556) (end 131.162 148.505) (width 0.2) (layer "B.Cu") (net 13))
 (segment (start 132.436 148.505) (end 132.948 149.017) (width 0.2) (layer "B.Cu") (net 13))
 (segment (start 115.54 148.65) (end 117.101 147.088) (width 0.2) (layer "B.Cu") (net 13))
 (segment (start 115.54 148.65) (end 114.318 148.65) (width 0.2) (layer "B.Cu") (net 13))
 (segment (start 132.948 150.829) (end 132.427 151.35) (width 0.2) (layer "B.Cu") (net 13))
 (segment (start 117.101 147.088) (end 130.695 147.088) (width 0.2) (layer "B.Cu") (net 13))
 (segment (start 119.556 148.306) (end 118.65 147.4) (width 0.2) (layer "F.Cu") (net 8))
 (segment (start 123.265 152.7) (end 123.265 151.043) (width 0.2) (layer "F.Cu") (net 8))
 (segment (start 129.15 147.2) (end 129.648 147.698) (width 0.2) (layer "F.Cu") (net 8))
 (segment (start 129.648 147.698) (end 130.159 147.698) (width 0.2) (layer "F.Cu") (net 8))
 (via (at 130.159 147.698) (size 0.6) (drill 0.3) (layers "F.Cu" "B.Cu") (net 8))
 (via (at 119.556 148.306) (size 0.6) (drill 0.3) (layers "F.Cu" "B.Cu") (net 8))
 (via (at 123.265 151.043) (size 0.6) (drill 0.3) (layers "F.Cu" "B.Cu") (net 8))
 (segment (start 123.265 151.043) (end 123.265 149.209) (width 0.2) (layer "B.Cu") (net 8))
 (segment (start 122.122 149.209) (end 123.265 149.209) (width 0.2) (layer "B.Cu") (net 8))
 (segment (start 130.159 147.698) (end 129.977 147.517) (width 0.2) (layer "B.Cu") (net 8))
 (segment (start 129.977 147.517) (end 124.957 147.517) (width 0.2) (layer "B.Cu") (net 8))
 (segment (start 124.957 147.517) (end 123.265 149.209) (width 0.2) (layer "B.Cu") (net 8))
 (segment (start 121.044 148.131) (end 122.122 149.209) (width 0.2) (layer "B.Cu") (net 8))
 (segment (start 119.556 148.306) (end 119.732 148.131) (width 0.2) (layer "B.Cu") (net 8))
 (segment (start 119.732 148.131) (end 121.044 148.131) (width 0.2) (layer "B.Cu") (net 8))
 (segment (start 122.197 149.244) (end 122.615 149.244) (width 0.2) (layer "F.Cu") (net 12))
 (segment (start 120.55 147.4) (end 120.55 147.597) (width 0.2) (layer "F.Cu") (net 12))
 (segment (start 122.615 149.244) (end 123.265 148.594) (width 0.2) (layer "F.Cu") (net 12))
 (segment (start 124.535 147.3) (end 123.265 147.3) (width 0.2) (layer "F.Cu") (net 12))
 (segment (start 120.55 147.597) (end 122.197 149.244) (width 0.2) (layer "F.Cu") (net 12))
 (segment (start 123.265 148.594) (end 123.265 147.3) (width 0.2) (layer "F.Cu") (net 12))
 (segment (start 129.22 149.943) (end 129.358 149.943) (width 0.2) (layer "F.Cu") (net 2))
 (segment (start 129.15 152.8) (end 129.15 151.764) (width 0.2) (layer "F.Cu") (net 2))
 (segment (start 119.564 151.686) (end 119.564 151.445) (width 0.2) (layer "F.Cu") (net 2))
 (segment (start 124.535 152.7) (end 124.676 152.559) (width 0.2) (layer "F.Cu") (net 2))
 (segment (start 128.277 150.887) (end 129.22 149.943) (width 0.2) (layer "F.Cu") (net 2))
 (segment (start 124.676 152.559) (end 124.676 151.406) (width 0.2) (layer "F.Cu") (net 2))
 (segment (start 129.15 151.764) (end 129.359 151.555) (width 0.2) (layer "F.Cu") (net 2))
 (segment (start 118.65 152.6) (end 119.564 151.686) (width 0.2) (layer "F.Cu") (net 2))
 (via (at 128.277 150.887) (size 0.6) (drill 0.3) (layers "F.Cu" "B.Cu") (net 2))
 (via (at 129.358 149.943) (size 0.6) (drill 0.3) (layers "F.Cu" "B.Cu") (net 2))
 (via (at 129.359 151.555) (size 0.6) (drill 0.3) (layers "F.Cu" "B.Cu") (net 2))
 (via (at 119.564 151.445) (size 0.6) (drill 0.3) (layers "F.Cu" "B.Cu") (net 2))
 (via (at 124.676 151.406) (size 0.6) (drill 0.3) (layers "F.Cu" "B.Cu") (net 2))
 (segment (start 128.945 151.555) (end 129.359 151.555) (width 0.2) (layer "B.Cu") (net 2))
 (segment (start 126.199 149.883) (end 129.298 149.883) (width 0.2) (layer "B.Cu") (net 2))
 (segment (start 129.298 149.883) (end 129.358 149.943) (width 0.2) (layer "B.Cu") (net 2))
 (segment (start 119.764 151.645) (end 119.564 151.445) (width 0.2) (layer "B.Cu") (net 2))
 (segment (start 124.676 151.406) (end 124.438 151.645) (width 0.2) (layer "B.Cu") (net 2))
 (segment (start 124.438 151.645) (end 119.764 151.645) (width 0.2) (layer "B.Cu") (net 2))
 (segment (start 124.676 151.406) (end 126.199 149.883) (width 0.2) (layer "B.Cu") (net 2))
 (segment (start 128.277 150.887) (end 128.945 151.555) (width 0.2) (layer "B.Cu") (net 2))
 (segment (start 125.805 151.569) (end 124.678 150.441) (width 0.2) (layer "F.Cu") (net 6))
 (segment (start 124.678 150.441) (end 122.028 150.441) (width 0.2) (layer "F.Cu") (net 6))
 (segment (start 120.55 151.92) (end 120.55 152.6) (width 0.2) (layer "F.Cu") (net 6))
 (segment (start 116.307 151.384) (end 116.307 151.443) (width 0.2) (layer "F.Cu") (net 6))
 (segment (start 116.307 151.443) (end 115.15 152.6) (width 0.2) (layer "F.Cu") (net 6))
 (segment (start 125.805 151.569) (end 126.372 151.569) (width 0.2) (layer "F.Cu") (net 6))
 (segment (start 125.805 152.7) (end 125.805 151.569) (width 0.2) (layer "F.Cu") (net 6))
 (segment (start 122.028 150.441) (end 120.55 151.92) (width 0.2) (layer "F.Cu") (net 6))
 (via (at 116.307 151.384) (size 0.6) (drill 0.3) (layers "F.Cu" "B.Cu") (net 6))
 (via (at 126.372 151.569) (size 0.6) (drill 0.3) (layers "F.Cu" "B.Cu") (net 6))
 (segment (start 114.62 151.602) (end 115.501 152.484) (width 0.2) (layer "B.Cu") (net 6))
 (segment (start 116.307 151.384) (end 115.622 150.698) (width 0.2) (layer "B.Cu") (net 6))
 (segment (start 114.62 151.074) (end 114.62 151.602) (width 0.2) (layer "B.Cu") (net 6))
 (segment (start 115.501 152.484) (end 125.458 152.484) (width 0.2) (layer "B.Cu") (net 6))
 (segment (start 125.458 152.484) (end 126.372 151.569) (width 0.2) (layer "B.Cu") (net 6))
 (segment (start 114.995 150.698) (end 114.62 151.074) (width 0.2) (layer "B.Cu") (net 6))
 (segment (start 115.622 150.698) (end 114.995 150.698) (width 0.2) (layer "B.Cu") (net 6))
 (segment (start 115.15 150) (end 115.15 149.822) (width 0.2) (layer "F.Cu") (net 3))
 (segment (start 121.995 147.3) (end 122.422 147.726) (width 0.2) (layer "F.Cu") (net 3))
 (segment (start 115.15 149.822) (end 114.139 149.822) (width 0.2) (layer "F.Cu") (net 3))
 (segment (start 121.572 150) (end 120.55 150) (width 0.2) (layer "F.Cu") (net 3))
 (segment (start 115.15 149.822) (end 115.15 148.669) (width 0.2) (layer "F.Cu") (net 3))
 (segment (start 115.15 148.669) (end 116.41 148.669) (width 0.2) (layer "F.Cu") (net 3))
 (segment (start 122.422 147.726) (end 122.422 148.585) (width 0.2) (layer "F.Cu") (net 3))
 (segment (start 115.15 148.669) (end 115.15 147.4) (width 0.2) (layer "F.Cu") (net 3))
 (via (at 121.572 150) (size 0.6) (drill 0.3) (layers "F.Cu" "B.Cu") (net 3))
 (via (at 114.139 149.822) (size 0.6) (drill 0.3) (layers "F.Cu" "B.Cu") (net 3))
 (via (at 122.422 148.585) (size 0.6) (drill 0.3) (layers "F.Cu" "B.Cu") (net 3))
 (via (at 116.41 148.669) (size 0.6) (drill 0.3) (layers "F.Cu" "B.Cu") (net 3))
 (segment (start 116.41 148.669) (end 117.383 147.696) (width 0.2) (layer "B.Cu") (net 3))
 (segment (start 121.394 149.822) (end 114.139 149.822) (width 0.2) (layer "B.Cu") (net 3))
 (segment (start 117.383 147.696) (end 121.532 147.696) (width 0.2) (layer "B.Cu") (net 3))
 (segment (start 121.572 150) (end 121.394 149.822) (width 0.2) (layer "B.Cu") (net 3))
 (segment (start 121.532 147.696) (end 122.422 148.585) (width 0.2) (layer "B.Cu") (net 3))
 (segment (start 110.1 152.6) (end 111.336 151.364) (width 0.2) (layer "F.Cu") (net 16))
 (segment (start 117.05 152.6) (end 118.28 151.37) (width 0.2) (layer "F.Cu") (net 16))
 (via (at 118.28 151.37) (size 0.6) (drill 0.3) (layers "F.Cu" "B.Cu") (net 16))
 (via (at 111.336 151.364) (size 0.6) (drill 0.3) (layers "F.Cu" "B.Cu") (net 16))
 (segment (start 113.644 151.449) (end 113.644 151.591) (width 0.2) (layer "B.Cu") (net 16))
 (segment (start 114.797 150.296) (end 113.644 151.449) (width 0.2) (layer "B.Cu") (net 16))
 (segment (start 118.28 151.37) (end 117.207 150.296) (width 0.2) (layer "B.Cu") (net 16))
 (segment (start 117.207 150.296) (end 114.797 150.296) (width 0.2) (layer "B.Cu") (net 16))
 (segment (start 112.898 152.337) (end 112.309 152.337) (width 0.2) (layer "B.Cu") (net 16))
 (segment (start 112.309 152.337) (end 111.336 151.364) (width 0.2) (layer "B.Cu") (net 16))
 (segment (start 113.644 151.591) (end 112.898 152.337) (width 0.2) (layer "B.Cu") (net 16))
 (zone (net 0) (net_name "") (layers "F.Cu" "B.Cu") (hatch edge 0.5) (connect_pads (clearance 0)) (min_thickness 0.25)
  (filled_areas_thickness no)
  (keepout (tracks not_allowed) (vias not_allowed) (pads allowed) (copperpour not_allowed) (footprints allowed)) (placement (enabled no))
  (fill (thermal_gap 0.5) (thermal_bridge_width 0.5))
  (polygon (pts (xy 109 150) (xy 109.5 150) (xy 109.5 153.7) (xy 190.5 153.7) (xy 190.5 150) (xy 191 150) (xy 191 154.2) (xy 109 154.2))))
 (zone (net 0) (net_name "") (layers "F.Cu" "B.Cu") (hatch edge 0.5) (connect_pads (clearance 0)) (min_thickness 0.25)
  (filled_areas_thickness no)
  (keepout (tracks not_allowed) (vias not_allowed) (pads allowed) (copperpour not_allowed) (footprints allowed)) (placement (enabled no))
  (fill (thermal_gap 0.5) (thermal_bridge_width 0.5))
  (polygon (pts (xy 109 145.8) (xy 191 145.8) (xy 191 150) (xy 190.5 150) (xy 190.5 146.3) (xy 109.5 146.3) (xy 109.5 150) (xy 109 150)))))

